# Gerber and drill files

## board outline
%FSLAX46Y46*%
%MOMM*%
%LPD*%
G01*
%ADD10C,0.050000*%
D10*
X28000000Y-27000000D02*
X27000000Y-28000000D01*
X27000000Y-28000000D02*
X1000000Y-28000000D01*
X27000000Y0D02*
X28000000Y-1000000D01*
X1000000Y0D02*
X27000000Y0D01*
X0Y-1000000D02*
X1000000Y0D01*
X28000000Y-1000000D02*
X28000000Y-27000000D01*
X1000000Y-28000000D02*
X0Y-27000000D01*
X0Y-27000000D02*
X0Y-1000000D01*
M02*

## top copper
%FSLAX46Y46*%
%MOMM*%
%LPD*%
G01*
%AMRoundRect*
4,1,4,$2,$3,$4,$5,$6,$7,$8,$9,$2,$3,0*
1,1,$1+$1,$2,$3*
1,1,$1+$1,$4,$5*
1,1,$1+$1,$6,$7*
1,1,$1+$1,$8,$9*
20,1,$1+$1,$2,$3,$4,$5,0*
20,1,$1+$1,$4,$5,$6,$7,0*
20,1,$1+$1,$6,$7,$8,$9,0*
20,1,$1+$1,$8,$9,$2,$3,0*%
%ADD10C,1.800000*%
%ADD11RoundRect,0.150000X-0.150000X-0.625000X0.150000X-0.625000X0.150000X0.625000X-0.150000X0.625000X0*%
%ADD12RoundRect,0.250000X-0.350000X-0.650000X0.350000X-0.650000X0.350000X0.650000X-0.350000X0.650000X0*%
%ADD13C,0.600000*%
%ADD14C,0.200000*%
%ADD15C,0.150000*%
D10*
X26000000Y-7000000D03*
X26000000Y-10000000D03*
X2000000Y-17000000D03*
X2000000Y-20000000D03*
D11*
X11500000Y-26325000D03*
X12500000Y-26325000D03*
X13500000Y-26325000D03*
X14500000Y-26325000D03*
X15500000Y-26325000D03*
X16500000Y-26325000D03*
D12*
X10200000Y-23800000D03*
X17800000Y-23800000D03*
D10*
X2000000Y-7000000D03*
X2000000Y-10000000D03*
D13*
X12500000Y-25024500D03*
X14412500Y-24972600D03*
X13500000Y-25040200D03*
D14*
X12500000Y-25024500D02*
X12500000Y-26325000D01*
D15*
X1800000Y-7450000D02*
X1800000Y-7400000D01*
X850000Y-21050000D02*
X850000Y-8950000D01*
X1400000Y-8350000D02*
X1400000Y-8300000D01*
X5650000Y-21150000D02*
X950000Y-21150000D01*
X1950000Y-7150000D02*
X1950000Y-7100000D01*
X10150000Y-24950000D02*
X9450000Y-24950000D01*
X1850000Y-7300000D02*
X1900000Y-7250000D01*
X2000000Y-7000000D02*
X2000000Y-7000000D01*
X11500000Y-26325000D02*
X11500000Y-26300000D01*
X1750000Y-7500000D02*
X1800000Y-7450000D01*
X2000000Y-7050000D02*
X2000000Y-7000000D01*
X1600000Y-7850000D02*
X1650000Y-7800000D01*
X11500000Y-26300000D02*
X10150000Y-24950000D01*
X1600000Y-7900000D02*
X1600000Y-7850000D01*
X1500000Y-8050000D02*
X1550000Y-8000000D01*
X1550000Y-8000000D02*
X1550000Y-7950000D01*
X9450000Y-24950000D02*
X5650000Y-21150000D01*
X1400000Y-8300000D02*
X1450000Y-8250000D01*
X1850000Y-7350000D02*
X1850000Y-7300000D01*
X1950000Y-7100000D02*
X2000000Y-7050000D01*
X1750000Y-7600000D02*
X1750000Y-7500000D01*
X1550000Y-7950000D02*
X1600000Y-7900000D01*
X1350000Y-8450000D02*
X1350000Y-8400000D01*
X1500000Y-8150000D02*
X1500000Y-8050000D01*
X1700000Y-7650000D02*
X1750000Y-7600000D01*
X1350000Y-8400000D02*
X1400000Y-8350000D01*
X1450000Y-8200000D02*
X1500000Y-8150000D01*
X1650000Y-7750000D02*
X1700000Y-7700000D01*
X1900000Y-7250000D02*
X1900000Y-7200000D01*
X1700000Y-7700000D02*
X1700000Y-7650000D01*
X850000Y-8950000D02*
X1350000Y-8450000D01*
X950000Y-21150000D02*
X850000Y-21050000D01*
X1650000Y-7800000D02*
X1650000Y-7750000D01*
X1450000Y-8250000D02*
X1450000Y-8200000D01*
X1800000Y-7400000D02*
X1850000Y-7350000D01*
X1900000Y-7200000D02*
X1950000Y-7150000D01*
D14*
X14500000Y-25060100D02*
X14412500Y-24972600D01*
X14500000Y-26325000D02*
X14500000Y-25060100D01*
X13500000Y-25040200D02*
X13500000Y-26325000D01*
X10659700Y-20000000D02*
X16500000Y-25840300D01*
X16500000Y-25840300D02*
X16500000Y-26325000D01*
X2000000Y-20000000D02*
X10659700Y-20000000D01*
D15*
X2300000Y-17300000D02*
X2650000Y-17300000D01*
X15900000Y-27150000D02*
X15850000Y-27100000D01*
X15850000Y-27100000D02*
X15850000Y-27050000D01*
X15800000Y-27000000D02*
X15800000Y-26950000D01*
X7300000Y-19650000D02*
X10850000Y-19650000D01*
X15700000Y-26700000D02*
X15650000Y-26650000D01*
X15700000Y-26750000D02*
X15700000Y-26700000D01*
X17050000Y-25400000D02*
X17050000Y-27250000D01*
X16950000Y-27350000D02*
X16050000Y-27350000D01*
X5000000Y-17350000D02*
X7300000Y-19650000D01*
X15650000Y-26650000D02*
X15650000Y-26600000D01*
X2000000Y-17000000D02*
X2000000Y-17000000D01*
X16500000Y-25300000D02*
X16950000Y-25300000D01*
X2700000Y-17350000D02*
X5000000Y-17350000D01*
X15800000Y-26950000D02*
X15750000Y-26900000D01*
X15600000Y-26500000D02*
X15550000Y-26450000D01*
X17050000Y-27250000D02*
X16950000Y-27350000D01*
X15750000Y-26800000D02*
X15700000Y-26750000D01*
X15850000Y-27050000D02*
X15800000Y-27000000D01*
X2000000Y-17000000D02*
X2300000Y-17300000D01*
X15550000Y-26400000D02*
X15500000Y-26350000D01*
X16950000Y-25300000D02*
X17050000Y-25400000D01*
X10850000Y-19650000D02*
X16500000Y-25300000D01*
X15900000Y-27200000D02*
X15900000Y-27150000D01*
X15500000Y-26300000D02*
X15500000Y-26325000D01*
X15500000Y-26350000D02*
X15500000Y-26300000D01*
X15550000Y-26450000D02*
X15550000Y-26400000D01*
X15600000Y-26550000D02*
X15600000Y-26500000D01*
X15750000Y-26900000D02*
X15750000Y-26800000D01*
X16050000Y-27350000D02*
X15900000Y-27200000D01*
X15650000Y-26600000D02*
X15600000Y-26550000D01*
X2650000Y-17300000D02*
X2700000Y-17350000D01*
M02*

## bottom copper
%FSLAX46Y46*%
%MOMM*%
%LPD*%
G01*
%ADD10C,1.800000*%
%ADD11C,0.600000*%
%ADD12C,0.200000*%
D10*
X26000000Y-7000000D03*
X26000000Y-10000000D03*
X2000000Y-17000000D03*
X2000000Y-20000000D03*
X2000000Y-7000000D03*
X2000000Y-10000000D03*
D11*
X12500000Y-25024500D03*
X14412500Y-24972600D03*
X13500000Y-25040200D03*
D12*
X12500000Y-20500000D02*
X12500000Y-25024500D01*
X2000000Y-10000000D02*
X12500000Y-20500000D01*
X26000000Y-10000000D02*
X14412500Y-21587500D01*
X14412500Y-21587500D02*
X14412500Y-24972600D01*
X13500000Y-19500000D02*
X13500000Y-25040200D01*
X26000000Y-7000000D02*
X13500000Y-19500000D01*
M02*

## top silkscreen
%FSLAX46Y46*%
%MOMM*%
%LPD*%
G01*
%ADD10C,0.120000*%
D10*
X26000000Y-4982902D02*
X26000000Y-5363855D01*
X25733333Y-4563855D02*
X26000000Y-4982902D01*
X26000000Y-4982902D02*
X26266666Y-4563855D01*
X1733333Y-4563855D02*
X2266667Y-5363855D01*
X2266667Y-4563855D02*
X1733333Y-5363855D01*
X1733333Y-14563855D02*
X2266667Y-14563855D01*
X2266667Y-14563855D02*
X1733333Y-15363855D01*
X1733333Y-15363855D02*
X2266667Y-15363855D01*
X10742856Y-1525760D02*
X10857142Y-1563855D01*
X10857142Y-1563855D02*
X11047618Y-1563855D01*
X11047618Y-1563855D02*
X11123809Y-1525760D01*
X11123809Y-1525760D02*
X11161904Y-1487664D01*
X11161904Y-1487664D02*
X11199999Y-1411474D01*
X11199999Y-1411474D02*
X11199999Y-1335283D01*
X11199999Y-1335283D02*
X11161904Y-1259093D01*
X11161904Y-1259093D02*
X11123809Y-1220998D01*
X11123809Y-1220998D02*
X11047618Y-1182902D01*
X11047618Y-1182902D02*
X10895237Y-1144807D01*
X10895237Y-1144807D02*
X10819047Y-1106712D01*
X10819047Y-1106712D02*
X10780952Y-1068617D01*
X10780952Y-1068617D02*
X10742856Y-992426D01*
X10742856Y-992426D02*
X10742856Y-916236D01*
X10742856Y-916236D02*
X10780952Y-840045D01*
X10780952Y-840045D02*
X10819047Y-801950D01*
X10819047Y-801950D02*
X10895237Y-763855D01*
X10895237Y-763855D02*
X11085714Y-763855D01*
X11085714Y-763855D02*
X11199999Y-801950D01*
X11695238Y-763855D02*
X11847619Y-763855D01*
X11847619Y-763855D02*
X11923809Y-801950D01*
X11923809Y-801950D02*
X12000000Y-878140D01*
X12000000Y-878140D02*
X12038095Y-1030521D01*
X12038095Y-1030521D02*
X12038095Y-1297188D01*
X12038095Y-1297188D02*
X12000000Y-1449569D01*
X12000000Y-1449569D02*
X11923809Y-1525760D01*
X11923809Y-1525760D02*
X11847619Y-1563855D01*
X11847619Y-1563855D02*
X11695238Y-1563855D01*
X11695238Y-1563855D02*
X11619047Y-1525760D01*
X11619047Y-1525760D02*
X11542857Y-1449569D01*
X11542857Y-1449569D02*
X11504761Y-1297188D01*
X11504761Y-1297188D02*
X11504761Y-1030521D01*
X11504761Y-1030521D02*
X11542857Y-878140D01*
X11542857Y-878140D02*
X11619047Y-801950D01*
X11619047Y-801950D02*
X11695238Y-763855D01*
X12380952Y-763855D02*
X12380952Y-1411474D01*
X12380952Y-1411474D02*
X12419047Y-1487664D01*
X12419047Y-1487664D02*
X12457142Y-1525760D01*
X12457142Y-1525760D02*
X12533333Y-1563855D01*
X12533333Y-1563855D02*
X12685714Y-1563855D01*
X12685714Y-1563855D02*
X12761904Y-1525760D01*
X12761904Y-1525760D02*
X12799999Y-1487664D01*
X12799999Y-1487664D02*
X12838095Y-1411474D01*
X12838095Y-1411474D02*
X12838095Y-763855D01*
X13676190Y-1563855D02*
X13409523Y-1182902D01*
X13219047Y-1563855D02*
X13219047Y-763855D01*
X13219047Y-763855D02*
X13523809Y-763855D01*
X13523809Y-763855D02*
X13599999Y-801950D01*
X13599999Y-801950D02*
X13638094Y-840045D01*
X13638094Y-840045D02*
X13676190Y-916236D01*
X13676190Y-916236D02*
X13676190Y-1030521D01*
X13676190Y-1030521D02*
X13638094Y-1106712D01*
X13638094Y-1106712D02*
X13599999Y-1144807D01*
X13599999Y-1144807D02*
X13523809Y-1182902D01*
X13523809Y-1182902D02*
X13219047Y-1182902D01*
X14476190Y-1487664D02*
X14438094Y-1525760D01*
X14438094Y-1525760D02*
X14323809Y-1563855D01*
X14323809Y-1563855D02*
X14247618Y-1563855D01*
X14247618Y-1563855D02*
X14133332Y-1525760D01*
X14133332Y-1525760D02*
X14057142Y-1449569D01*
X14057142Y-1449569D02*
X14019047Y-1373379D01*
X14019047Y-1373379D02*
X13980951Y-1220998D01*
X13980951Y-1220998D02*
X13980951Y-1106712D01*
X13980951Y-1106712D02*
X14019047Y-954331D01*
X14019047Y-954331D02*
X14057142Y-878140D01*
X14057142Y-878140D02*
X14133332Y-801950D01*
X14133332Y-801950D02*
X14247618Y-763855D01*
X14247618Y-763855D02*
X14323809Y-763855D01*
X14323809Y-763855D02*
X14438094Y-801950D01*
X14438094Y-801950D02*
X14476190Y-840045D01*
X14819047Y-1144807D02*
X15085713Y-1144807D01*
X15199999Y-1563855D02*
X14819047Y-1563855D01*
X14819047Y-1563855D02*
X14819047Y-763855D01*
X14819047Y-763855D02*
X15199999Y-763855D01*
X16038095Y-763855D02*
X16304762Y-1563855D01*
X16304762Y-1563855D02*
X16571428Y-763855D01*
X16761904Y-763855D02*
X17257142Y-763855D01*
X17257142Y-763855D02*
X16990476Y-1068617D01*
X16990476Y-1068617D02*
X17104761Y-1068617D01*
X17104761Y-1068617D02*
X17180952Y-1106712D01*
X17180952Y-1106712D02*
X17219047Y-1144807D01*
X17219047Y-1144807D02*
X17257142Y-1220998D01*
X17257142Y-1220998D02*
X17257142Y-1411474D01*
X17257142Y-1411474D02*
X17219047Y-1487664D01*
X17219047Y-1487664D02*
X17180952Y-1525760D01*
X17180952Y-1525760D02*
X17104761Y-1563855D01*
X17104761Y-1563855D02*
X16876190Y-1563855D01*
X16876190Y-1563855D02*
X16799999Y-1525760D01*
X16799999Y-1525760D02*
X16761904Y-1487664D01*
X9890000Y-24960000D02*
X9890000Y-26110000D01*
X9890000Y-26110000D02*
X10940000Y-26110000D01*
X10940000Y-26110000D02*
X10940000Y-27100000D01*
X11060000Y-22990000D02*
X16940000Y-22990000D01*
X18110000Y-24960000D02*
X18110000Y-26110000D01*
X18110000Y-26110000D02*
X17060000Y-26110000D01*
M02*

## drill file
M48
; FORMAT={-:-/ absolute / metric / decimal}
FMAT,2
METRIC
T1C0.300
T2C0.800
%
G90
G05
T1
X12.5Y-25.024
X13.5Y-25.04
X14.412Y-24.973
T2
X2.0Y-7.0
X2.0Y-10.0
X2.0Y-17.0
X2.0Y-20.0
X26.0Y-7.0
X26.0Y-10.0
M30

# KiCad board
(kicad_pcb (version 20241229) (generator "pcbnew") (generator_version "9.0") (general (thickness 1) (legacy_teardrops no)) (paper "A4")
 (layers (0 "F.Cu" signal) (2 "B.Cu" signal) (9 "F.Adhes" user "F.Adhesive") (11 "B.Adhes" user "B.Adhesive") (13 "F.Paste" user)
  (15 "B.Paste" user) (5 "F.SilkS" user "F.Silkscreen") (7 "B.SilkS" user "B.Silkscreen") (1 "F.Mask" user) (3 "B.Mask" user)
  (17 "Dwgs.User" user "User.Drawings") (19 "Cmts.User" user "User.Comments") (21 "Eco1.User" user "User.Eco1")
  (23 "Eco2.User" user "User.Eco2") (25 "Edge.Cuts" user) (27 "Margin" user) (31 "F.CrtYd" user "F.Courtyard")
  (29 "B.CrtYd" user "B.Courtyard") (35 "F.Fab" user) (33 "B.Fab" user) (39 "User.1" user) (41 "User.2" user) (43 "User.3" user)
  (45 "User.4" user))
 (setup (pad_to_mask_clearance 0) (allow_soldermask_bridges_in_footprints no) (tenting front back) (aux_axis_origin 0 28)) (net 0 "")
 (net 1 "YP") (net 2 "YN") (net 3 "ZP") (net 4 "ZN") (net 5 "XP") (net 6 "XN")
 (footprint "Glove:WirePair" (layer "F.Cu") (at 26 7)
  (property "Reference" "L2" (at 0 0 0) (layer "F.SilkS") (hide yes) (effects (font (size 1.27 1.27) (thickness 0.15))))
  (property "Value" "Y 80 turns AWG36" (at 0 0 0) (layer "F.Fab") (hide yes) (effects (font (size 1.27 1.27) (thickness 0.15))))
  (pad "1" thru_hole circle (at 0 0) (size 1.8 1.8) (drill 0.8) (layers "*.Cu" "*.Mask") (remove_unused_layers no) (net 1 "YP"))
  (pad "2" thru_hole circle (at 0 3) (size 1.8 1.8) (drill 0.8) (layers "*.Cu" "*.Mask") (remove_unused_layers no) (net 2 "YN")))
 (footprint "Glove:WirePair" (layer "F.Cu") (at 2 17)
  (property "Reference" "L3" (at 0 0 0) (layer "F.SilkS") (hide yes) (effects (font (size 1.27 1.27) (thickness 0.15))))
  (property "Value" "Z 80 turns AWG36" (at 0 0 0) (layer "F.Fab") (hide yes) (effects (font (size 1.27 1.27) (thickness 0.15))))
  (pad "1" thru_hole circle (at 0 0) (size 1.8 1.8) (drill 0.8) (layers "*.Cu" "*.Mask") (remove_unused_layers no) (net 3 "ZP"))
  (pad "2" thru_hole circle (at 0 3) (size 1.8 1.8) (drill 0.8) (layers "*.Cu" "*.Mask") (remove_unused_layers no) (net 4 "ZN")))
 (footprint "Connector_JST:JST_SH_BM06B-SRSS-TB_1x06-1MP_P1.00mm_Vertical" (layer "F.Cu") (at 14 25)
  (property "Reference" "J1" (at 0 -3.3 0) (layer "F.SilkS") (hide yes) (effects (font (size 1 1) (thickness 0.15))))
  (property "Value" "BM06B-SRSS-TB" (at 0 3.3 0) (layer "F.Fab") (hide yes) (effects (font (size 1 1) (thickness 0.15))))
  (fp_line (start -4.11 -0.04) (end -4.11 1.11) (stroke (width 0.12) (type solid)) (layer "F.SilkS"))
  (fp_line (start -4.11 1.11) (end -3.06 1.11) (stroke (width 0.12) (type solid)) (layer "F.SilkS"))
  (fp_line (start -3.06 1.11) (end -3.06 2.1) (stroke (width 0.12) (type solid)) (layer "F.SilkS"))
  (fp_line (start -2.94 -2.01) (end 2.94 -2.01) (stroke (width 0.12) (type solid)) (layer "F.SilkS"))
  (fp_line (start 4.11 -0.04) (end 4.11 1.11) (stroke (width 0.12) (type solid)) (layer "F.SilkS"))
  (fp_line (start 4.11 1.11) (end 3.06 1.11) (stroke (width 0.12) (type solid)) (layer "F.SilkS"))
  (pad "1" smd roundrect (at -2.5 1.325) (size 0.6 1.55) (layers "F.Cu" "F.Mask" "F.Paste") (roundrect_rratio 0.25) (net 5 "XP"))
  (pad "2" smd roundrect (at -1.5 1.325) (size 0.6 1.55) (layers "F.Cu" "F.Mask" "F.Paste") (roundrect_rratio 0.25) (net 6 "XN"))
  (pad "3" smd roundrect (at -0.5 1.325) (size 0.6 1.55) (layers "F.Cu" "F.Mask" "F.Paste") (roundrect_rratio 0.25) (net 1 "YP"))
  (pad "4" smd roundrect (at 0.5 1.325) (size 0.6 1.55) (layers "F.Cu" "F.Mask" "F.Paste") (roundrect_rratio 0.25) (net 2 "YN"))
  (pad "5" smd roundrect (at 1.5 1.325) (size 0.6 1.55) (layers "F.Cu" "F.Mask" "F.Paste") (roundrect_rratio 0.25) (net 3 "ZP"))
  (pad "6" smd roundrect (at 2.5 1.325) (size 0.6 1.55) (layers "F.Cu" "F.Mask" "F.Paste") (roundrect_rratio 0.25) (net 4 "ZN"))
  (pad "MP" smd roundrect (at -3.8 -1.2) (size 1.2 1.8) (layers "F.Cu" "F.Mask" "F.Paste") (roundrect_rratio 0.208333))
  (pad "MP" smd roundrect (at 3.8 -1.2) (size 1.2 1.8) (layers "F.Cu" "F.Mask" "F.Paste") (roundrect_rratio 0.208333)))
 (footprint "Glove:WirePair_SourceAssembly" (layer "F.Cu") (at 2 7)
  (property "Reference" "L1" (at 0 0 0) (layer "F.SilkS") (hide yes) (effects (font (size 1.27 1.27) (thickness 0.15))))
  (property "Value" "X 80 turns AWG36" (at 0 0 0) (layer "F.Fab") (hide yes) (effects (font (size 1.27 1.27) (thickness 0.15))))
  (pad "1" thru_hole circle (at 0 0) (size 1.8 1.8) (drill 0.8) (layers "*.Cu" "*.Mask") (remove_unused_layers no) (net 5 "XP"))
  (pad "2" thru_hole circle (at 0 3) (size 1.8 1.8) (drill 0.8) (layers "*.Cu" "*.Mask") (remove_unused_layers no) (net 6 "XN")))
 (gr_line (start 28 27) (end 27 28) (stroke (width 0.05) (type default)) (layer "Edge.Cuts"))
 (gr_line (start 27 28) (end 1 28) (stroke (width 0.05) (type default)) (layer "Edge.Cuts"))
 (gr_line (start 27 0) (end 28 1) (stroke (width 0.05) (type default)) (layer "Edge.Cuts"))
 (gr_line (start 1 0) (end 27 0) (stroke (width 0.05) (type default)) (layer "Edge.Cuts"))
 (gr_line (start 0 1) (end 1 0) (stroke (width 0.05) (type default)) (layer "Edge.Cuts"))
 (gr_line (start 28 1) (end 28 27) (stroke (width 0.05) (type default)) (layer "Edge.Cuts"))
 (gr_line (start 1 28) (end 0 27) (stroke (width 0.05) (type default)) (layer "Edge.Cuts"))
 (gr_line (start 0 27) (end 0 1) (stroke (width 0.05) (type default)) (layer "Edge.Cuts"))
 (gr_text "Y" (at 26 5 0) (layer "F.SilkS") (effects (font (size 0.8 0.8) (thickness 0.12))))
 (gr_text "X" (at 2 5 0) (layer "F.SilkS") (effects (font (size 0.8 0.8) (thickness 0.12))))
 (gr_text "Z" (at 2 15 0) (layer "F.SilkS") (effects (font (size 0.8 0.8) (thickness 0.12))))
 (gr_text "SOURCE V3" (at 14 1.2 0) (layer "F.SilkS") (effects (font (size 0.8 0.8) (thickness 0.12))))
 (segment (start 12.5 25.0245) (end 12.5 26.325) (width 0.2) (layer "F.Cu") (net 6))
 (via (at 12.5 25.0245) (size 0.6) (drill 0.3) (layers "F.Cu" "B.Cu") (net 6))
 (segment (start 12.5 20.5) (end 12.5 25.0245) (width 0.2) (layer "B.Cu") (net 6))
 (segment (start 2 10) (end 12.5 20.5) (width 0.2) (layer "B.Cu") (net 6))
 (segment (start 1.8 7.45) (end 1.8 7.4) (width 0.15) (layer "F.Cu") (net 5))
 (segment (start 0.85 21.05) (end 0.85 8.95) (width 0.15) (layer "F.Cu") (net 5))
 (segment (start 1.4 8.35) (end 1.4 8.3) (width 0.15) (layer "F.Cu") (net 5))
 (segment (start 5.65 21.15) (end 0.95 21.15) (width 0.15) (layer "F.Cu") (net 5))
 (segment (start 1.95 7.15) (end 1.95 7.1) (width 0.15) (layer "F.Cu") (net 5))
 (segment (start 10.15 24.95) (end 9.45 24.95) (width 0.15) (layer "F.Cu") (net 5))
 (segment (start 1.85 7.3) (end 1.9 7.25) (width 0.15) (layer "F.Cu") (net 5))
 (segment (start 2 7) (end 2 7) (width 0.15) (layer "F.Cu") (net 5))
 (segment (start 11.5 26.325) (end 11.5 26.3) (width 0.15) (layer "F.Cu") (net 5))
 (segment (start 1.75 7.5) (end 1.8 7.45) (width 0.15) (layer "F.Cu") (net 5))
 (segment (start 2 7.05) (end 2 7) (width 0.15) (layer "F.Cu") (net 5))
 (segment (start 1.6 7.85) (end 1.65 7.8) (width 0.15) (layer "F.Cu") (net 5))
 (segment (start 11.5 26.3) (end 10.15 24.95) (width 0.15) (layer "F.Cu") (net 5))
 (segment (start 1.6 7.9) (end 1.6 7.85) (width 0.15) (layer "F.Cu") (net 5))
 (segment (start 1.5 8.05) (end 1.55 8) (width 0.15) (layer "F.Cu") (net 5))
 (segment (start 1.55 8) (end 1.55 7.95) (width 0.15) (layer "F.Cu") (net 5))
 (segment (start 9.45 24.95) (end 5.65 21.15) (width 0.15) (layer "F.Cu") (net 5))
 (segment (start 1.4 8.3) (end 1.45 8.25) (width 0.15) (layer "F.Cu") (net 5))
 (segment (start 1.85 7.35) (end 1.85 7.3) (width 0.15) (layer "F.Cu") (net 5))
 (segment (start 1.95 7.1) (end 2 7.05) (width 0.15) (layer "F.Cu") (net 5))
 (segment (start 1.75 7.6) (end 1.75 7.5) (width 0.15) (layer "F.Cu") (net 5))
 (segment (start 1.55 7.95) (end 1.6 7.9) (width 0.15) (layer "F.Cu") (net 5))
 (segment (start 1.35 8.45) (end 1.35 8.4) (width 0.15) (layer "F.Cu") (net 5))
 (segment (start 1.5 8.15) (end 1.5 8.05) (width 0.15) (layer "F.Cu") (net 5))
 (segment (start 1.7 7.65) (end 1.75 7.6) (width 0.15) (layer "F.Cu") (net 5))
 (segment (start 1.35 8.4) (end 1.4 8.35) (width 0.15) (layer "F.Cu") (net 5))
 (segment (start 1.45 8.2) (end 1.5 8.15) (width 0.15) (layer "F.Cu") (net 5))
 (segment (start 1.65 7.75) (end 1.7 7.7) (width 0.15) (layer "F.Cu") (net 5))
 (segment (start 1.9 7.25) (end 1.9 7.2) (width 0.15) (layer "F.Cu") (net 5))
 (segment (start 1.7 7.7) (end 1.7 7.65) (width 0.15) (layer "F.Cu") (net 5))
 (segment (start 0.85 8.95) (end 1.35 8.45) (width 0.15) (layer "F.Cu") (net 5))
 (segment (start 0.95 21.15) (end 0.85 21.05) (width 0.15) (layer "F.Cu") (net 5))
 (segment (start 1.65 7.8) (end 1.65 7.75) (width 0.15) (layer "F.Cu") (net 5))
 (segment (start 1.45 8.25) (end 1.45 8.2) (width 0.15) (layer "F.Cu") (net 5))
 (segment (start 1.8 7.4) (end 1.85 7.35) (width 0.15) (layer "F.Cu") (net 5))
 (segment (start 1.9 7.2) (end 1.95 7.15) (width 0.15) (layer "F.Cu") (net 5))
 (segment (start 14.5 25.0601) (end 14.4125 24.9726) (width 0.2) (layer "F.Cu") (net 2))
 (segment (start 14.5 26.325) (end 14.5 25.0601) (width 0.2) (layer "F.Cu") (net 2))
 (via (at 14.4125 24.9726) (size 0.6) (drill 0.3) (layers "F.Cu" "B.Cu") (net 2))
 (segment (start 26 10) (end 14.4125 21.5875) (width 0.2) (layer "B.Cu") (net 2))
 (segment (start 14.4125 21.5875) (end 14.4125 24.9726) (width 0.2) (layer "B.Cu") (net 2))
 (segment (start 13.5 25.0402) (end 13.5 26.325) (width 0.2) (layer "F.Cu") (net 1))
 (via (at 13.5 25.0402) (size 0.6) (drill 0.3) (layers "F.Cu" "B.Cu") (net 1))
 (segment (start 13.5 19.5) (end 13.5 25.0402) (width 0.2) (layer "B.Cu") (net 1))
 (segment (start 26 7) (end 13.5 19.5) (width 0.2) (layer "B.Cu") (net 1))
 (segment (start 10.6597 20) (end 16.5 25.8403) (width 0.2) (layer "F.Cu") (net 4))
 (segment (start 16.5 25.8403) (end 16.5 26.325) (width 0.2) (layer "F.Cu") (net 4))
 (segment (start 2 20) (end 10.6597 20) (width 0.2) (layer "F.Cu") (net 4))
 (segment (start 2.3 17.3) (end 2.65 17.3) (width 0.15) (layer "F.Cu") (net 3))
 (segment (start 15.9 27.15) (end 15.85 27.1) (width 0.15) (layer "F.Cu") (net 3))
 (segment (start 15.85 27.1) (end 15.85 27.05) (width 0.15) (layer "F.Cu") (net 3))
 (segment (start 15.8 27) (end 15.8 26.95) (width 0.15) (layer "F.Cu") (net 3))
 (segment (start 7.3 19.65) (end 10.85 19.65) (width 0.15) (layer "F.Cu") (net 3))
 (segment (start 15.7 26.7) (end 15.65 26.65) (width 0.15) (layer "F.Cu") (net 3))
 (segment (start 15.7 26.75) (end 15.7 26.7) (width 0.15) (layer "F.Cu") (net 3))
 (segment (start 17.05 25.4) (end 17.05 27.25) (width 0.15) (layer "F.Cu") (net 3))
 (segment (start 16.95 27.35) (end 16.05 27.35) (width 0.15) (layer "F.Cu") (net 3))
 (segment (start 5 17.35) (end 7.3 19.65) (width 0.15) (layer "F.Cu") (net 3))
 (segment (start 15.65 26.65) (end 15.65 26.6) (width 0.15) (layer "F.Cu") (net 3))
 (segment (start 2 17) (end 2 17) (width 0.15) (layer "F.Cu") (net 3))
 (segment (start 16.5 25.3) (end 16.95 25.3) (width 0.15) (layer "F.Cu") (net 3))
 (segment (start 2.7 17.35) (end 5 17.35) (width 0.15) (layer "F.Cu") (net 3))
 (segment (start 15.8 26.95) (end 15.75 26.9) (width 0.15) (layer "F.Cu") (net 3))
 (segment (start 15.6 26.5) (end 15.55 26.45) (width 0.15) (layer "F.Cu") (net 3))
 (segment (start 17.05 27.25) (end 16.95 27.35) (width 0.15) (layer "F.Cu") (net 3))
 (segment (start 15.75 26.8) (end 15.7 26.75) (width 0.15) (layer "F.Cu") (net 3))
 (segment (start 15.85 27.05) (end 15.8 27) (width 0.15) (layer "F.Cu") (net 3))
 (segment (start 2 17) (end 2.3 17.3) (width 0.15) (layer "F.Cu") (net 3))
 (segment (start 15.55 26.4) (end 15.5 26.35) (width 0.15) (layer "F.Cu") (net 3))
 (segment (start 16.95 25.3) (end 17.05 25.4) (width 0.15) (layer "F.Cu") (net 3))
 (segment (start 10.85 19.65) (end 16.5 25.3) (width 0.15) (layer "F.Cu") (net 3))
 (segment (start 15.9 27.2) (end 15.9 27.15) (width 0.15) (layer "F.Cu") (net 3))
 (segment (start 15.5 26.3) (end 15.5 26.325) (width 0.15) (layer "F.Cu") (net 3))
 (segment (start 15.5 26.35) (end 15.5 26.3) (width 0.15) (layer "F.Cu") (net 3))
 (segment (start 15.55 26.45) (end 15.55 26.4) (width 0.15) (layer "F.Cu") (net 3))
 (segment (start 15.6 26.55) (end 15.6 26.5) (width 0.15) (layer "F.Cu") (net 3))
 (segment (start 15.75 26.9) (end 15.75 26.8) (width 0.15) (layer "F.Cu") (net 3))
 (segment (start 16.05 27.35) (end 15.9 27.2) (width 0.15) (layer "F.Cu") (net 3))
 (segment (start 15.65 26.6) (end 15.6 26.55) (width 0.15) (layer "F.Cu") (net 3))
 (segment (start 2.65 17.3) (end 2.7 17.35) (width 0.15) (layer "F.Cu") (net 3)))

